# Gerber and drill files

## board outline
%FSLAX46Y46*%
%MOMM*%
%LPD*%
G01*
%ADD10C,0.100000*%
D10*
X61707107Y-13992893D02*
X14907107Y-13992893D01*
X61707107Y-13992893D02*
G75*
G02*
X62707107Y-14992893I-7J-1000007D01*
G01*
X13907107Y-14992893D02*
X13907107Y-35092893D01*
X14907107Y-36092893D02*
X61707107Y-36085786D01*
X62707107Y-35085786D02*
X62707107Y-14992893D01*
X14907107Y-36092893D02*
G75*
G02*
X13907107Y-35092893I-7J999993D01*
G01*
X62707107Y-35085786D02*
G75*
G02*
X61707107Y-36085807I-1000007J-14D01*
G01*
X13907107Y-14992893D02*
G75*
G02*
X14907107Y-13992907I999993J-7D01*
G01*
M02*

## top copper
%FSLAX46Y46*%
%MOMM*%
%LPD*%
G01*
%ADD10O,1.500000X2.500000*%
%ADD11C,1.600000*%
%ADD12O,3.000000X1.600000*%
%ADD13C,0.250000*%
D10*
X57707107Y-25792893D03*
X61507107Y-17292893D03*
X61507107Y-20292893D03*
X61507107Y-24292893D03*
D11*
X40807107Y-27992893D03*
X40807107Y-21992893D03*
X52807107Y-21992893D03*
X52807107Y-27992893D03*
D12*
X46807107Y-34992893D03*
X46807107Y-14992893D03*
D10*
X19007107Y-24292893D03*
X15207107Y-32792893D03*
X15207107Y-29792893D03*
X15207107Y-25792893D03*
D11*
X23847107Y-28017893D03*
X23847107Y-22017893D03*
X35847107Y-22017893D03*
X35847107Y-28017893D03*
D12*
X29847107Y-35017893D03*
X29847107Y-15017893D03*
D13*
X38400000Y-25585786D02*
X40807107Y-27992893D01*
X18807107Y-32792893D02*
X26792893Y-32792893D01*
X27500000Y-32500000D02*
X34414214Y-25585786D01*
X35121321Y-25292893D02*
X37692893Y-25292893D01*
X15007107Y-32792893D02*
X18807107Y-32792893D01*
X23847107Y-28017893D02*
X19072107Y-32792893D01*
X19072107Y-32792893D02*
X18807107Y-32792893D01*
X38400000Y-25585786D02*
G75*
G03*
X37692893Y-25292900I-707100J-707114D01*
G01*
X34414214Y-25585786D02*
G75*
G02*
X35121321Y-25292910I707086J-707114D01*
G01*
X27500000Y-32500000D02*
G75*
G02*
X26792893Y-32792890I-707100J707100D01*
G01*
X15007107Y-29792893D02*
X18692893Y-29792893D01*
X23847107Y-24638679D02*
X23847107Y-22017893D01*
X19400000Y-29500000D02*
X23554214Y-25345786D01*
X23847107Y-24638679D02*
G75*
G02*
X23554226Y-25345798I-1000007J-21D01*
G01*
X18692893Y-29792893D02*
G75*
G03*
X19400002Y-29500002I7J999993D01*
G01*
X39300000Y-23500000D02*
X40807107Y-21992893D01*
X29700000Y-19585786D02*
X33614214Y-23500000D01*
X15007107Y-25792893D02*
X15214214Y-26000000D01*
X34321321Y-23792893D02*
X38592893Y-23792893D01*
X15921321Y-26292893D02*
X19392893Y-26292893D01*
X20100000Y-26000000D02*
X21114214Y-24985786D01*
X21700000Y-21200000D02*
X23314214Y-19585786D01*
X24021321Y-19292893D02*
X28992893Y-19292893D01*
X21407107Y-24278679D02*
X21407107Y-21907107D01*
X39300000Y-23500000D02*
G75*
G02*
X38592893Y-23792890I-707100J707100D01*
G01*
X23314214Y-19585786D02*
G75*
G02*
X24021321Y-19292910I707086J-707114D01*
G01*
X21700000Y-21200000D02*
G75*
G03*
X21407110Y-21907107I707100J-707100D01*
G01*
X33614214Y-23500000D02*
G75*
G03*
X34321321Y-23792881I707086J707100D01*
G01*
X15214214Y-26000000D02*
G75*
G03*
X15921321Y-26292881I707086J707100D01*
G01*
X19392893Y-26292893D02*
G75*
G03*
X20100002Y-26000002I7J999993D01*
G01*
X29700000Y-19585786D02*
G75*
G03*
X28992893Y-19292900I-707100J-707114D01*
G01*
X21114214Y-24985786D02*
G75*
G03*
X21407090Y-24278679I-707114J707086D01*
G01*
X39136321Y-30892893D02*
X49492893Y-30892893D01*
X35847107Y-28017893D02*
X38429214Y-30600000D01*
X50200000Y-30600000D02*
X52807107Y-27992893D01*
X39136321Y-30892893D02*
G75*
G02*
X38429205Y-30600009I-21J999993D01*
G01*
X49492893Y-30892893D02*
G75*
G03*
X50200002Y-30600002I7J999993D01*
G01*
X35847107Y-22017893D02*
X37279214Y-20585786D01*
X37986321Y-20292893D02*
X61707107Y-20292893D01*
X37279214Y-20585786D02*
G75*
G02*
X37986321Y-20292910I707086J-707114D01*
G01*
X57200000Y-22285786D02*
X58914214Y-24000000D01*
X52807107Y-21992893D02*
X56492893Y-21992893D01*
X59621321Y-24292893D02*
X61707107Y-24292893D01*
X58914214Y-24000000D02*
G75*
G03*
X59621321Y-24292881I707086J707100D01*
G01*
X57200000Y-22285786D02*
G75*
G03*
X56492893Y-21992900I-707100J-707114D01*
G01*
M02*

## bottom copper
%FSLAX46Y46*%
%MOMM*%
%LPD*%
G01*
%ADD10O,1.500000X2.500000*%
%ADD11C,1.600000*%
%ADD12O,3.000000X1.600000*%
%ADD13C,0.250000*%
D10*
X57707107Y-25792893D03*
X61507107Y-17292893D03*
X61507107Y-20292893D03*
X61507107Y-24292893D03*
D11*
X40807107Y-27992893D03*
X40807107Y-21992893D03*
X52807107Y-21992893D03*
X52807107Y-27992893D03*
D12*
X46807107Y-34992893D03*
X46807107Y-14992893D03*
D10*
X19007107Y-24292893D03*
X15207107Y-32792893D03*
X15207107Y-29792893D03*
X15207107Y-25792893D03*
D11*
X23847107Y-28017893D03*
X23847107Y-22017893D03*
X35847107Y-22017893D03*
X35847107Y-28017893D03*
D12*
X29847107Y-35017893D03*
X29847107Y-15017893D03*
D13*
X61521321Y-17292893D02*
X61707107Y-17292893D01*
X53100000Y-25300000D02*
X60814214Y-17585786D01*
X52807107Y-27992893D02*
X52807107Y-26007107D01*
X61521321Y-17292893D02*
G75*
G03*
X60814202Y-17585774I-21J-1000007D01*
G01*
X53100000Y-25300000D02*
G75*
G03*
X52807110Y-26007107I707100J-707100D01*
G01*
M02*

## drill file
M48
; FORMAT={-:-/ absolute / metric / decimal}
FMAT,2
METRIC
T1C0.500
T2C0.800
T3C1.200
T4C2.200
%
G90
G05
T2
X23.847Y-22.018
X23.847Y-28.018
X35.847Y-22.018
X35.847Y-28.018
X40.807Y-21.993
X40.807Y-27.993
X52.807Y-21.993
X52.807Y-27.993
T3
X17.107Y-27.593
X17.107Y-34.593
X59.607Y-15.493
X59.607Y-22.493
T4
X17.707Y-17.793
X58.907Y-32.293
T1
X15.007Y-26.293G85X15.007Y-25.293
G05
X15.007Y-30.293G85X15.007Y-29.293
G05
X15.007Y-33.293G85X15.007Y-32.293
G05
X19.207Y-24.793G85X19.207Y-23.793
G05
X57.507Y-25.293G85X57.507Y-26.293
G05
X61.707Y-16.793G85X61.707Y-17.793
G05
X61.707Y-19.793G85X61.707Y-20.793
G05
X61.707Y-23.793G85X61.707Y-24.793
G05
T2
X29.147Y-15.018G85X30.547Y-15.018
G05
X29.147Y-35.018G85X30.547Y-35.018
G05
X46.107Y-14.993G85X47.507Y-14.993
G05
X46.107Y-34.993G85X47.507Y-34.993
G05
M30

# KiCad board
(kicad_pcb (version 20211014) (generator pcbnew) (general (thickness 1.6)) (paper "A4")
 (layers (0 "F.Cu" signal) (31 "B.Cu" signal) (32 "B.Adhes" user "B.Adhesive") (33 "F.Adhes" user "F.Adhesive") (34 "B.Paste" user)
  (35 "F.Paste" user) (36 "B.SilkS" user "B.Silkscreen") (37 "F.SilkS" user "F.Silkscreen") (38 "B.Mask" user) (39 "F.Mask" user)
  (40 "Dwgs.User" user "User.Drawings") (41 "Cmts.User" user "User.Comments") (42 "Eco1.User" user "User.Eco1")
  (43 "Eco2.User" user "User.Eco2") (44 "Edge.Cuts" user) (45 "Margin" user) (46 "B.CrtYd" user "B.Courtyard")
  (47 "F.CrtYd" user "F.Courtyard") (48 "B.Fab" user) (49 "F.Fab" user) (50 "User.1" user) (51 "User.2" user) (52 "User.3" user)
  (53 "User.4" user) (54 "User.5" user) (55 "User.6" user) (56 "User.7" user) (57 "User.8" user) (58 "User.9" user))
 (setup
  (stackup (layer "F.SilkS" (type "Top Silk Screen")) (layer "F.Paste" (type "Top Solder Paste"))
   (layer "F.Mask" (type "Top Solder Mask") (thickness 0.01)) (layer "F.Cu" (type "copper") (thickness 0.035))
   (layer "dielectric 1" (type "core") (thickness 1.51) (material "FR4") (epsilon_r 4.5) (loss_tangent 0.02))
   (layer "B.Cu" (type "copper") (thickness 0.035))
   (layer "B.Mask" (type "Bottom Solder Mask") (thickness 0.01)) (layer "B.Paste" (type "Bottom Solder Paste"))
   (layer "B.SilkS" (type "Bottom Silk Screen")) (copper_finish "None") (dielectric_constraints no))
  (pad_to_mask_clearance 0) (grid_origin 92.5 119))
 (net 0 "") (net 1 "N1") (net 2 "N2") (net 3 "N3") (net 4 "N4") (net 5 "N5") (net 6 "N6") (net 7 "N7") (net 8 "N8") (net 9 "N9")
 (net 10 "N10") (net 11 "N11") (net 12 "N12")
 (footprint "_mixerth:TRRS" (layer "F.Cu") (at 59.607107 13.992893)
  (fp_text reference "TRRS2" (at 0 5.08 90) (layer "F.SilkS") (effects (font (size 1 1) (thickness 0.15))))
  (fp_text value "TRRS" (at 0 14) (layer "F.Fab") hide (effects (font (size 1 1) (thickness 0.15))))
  (pad "" np_thru_hole circle (at 0 1.5) (size 1.2 1.2) (drill 1.2) (layers *.Cu *.Mask))
  (pad "" np_thru_hole circle (at 0 8.5) (size 1.2 1.2) (drill 1.2) (layers *.Cu *.Mask))
  (pad "A" thru_hole oval (at -2.1 11.8) (size 1.5 2.5) (drill oval 0.5 1.5 (offset 0.2 0)) (layers *.Cu "B.Mask") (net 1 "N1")
   (clearance 0.15))
  (pad "B" thru_hole oval (at 2.1 3.3) (size 1.5 2.5) (drill oval 0.5 1.5 (offset -0.2 0)) (layers *.Cu "B.Mask") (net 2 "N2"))
  (pad "C" thru_hole oval (at 2.1 6.3) (size 1.5 2.5) (drill oval 0.5 1.5 (offset -0.2 0)) (layers *.Cu "B.Mask") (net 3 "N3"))
  (pad "D" thru_hole oval (at 2.1 10.3) (size 1.5 2.5) (drill oval 0.5 1.5 (offset -0.2 0)) (layers *.Cu "B.Mask") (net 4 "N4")
   (clearance 0.15)))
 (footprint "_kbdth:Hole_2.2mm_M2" (layer "F.Cu") (at 58.907107 32.292893 90)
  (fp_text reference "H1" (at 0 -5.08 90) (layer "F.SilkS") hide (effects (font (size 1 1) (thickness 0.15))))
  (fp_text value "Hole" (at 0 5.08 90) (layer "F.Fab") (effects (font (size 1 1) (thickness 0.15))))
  (pad "" np_thru_hole circle locked (at 0 0 90) (size 2.2 2.2) (drill 2.2) (layers *.Cu *.Mask)))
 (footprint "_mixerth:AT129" (layer "F.Cu") (at 46.807107 24.992893 90)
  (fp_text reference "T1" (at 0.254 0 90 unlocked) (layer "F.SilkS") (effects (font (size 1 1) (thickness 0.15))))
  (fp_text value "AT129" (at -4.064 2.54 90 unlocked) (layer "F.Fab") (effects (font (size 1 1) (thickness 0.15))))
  (pad "1" thru_hole circle (at -3 -6 90) (size 1.6 1.6) (drill 0.8) (layers *.Cu "B.Mask") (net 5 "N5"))
  (pad "2" thru_hole circle (at 3 -6 90) (size 1.6 1.6) (drill 0.8) (layers *.Cu "B.Mask") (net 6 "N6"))
  (pad "3" thru_hole circle (at 3 6 90) (size 1.6 1.6) (drill 0.8) (layers *.Cu "B.Mask") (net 4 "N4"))
  (pad "4" thru_hole circle (at -3 6 90) (size 1.6 1.6) (drill 0.8) (layers *.Cu "B.Mask") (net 2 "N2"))
  (pad "5" thru_hole oval (at -10 0 90) (size 1.6 3) (drill oval 0.8 2.2) (layers *.Cu "B.Mask") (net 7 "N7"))
  (pad "6" thru_hole oval (at 10 0 90) (size 1.6 3) (drill oval 0.8 2.2) (layers *.Cu "B.Mask") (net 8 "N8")))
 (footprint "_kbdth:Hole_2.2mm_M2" (layer "F.Cu") (at 17.707107 17.792893 90)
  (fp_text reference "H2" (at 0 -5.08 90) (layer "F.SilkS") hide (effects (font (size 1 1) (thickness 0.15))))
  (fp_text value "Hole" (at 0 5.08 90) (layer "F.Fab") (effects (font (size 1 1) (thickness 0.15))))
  (pad "" np_thru_hole circle locked (at 0 0 90) (size 2.2 2.2) (drill 2.2) (layers *.Cu *.Mask)))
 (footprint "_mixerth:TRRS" (layer "F.Cu") (at 17.107107 36.092893 180)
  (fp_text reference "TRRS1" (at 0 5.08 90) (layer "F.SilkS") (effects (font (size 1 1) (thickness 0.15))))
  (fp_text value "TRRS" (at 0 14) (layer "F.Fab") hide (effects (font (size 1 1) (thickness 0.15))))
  (pad "" np_thru_hole circle (at 0 8.5 180) (size 1.2 1.2) (drill 1.2) (layers *.Cu *.Mask))
  (pad "" np_thru_hole circle (at 0 1.5 180) (size 1.2 1.2) (drill 1.2) (layers *.Cu *.Mask))
  (pad "A" thru_hole oval (at -2.1 11.8 180) (size 1.5 2.5) (drill oval 0.5 1.5 (offset 0.2 0)) (layers *.Cu "B.Mask") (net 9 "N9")
   (clearance 0.15))
  (pad "B" thru_hole oval (at 2.1 3.3 180) (size 1.5 2.5) (drill oval 0.5 1.5 (offset -0.2 0)) (layers *.Cu "B.Mask") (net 5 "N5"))
  (pad "C" thru_hole oval (at 2.1 6.3 180) (size 1.5 2.5) (drill oval 0.5 1.5 (offset -0.2 0)) (layers *.Cu "B.Mask") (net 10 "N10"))
  (pad "D" thru_hole oval (at 2.1 10.3 180) (size 1.5 2.5) (drill oval 0.5 1.5 (offset -0.2 0)) (layers *.Cu "B.Mask") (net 6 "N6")
   (clearance 0.15)))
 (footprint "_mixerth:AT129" (layer "F.Cu") (at 29.847107 25.017893 90)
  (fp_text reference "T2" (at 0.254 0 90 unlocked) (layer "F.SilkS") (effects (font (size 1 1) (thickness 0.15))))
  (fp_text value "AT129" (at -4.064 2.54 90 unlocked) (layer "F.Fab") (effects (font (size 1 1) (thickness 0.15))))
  (pad "1" thru_hole circle (at -3 -6 90) (size 1.6 1.6) (drill 0.8) (layers *.Cu "B.Mask") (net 5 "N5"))
  (pad "2" thru_hole circle (at 3 -6 90) (size 1.6 1.6) (drill 0.8) (layers *.Cu "B.Mask") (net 10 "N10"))
  (pad "3" thru_hole circle (at 3 6 90) (size 1.6 1.6) (drill 0.8) (layers *.Cu "B.Mask") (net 3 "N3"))
  (pad "4" thru_hole circle (at -3 6 90) (size 1.6 1.6) (drill 0.8) (layers *.Cu "B.Mask") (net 2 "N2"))
  (pad "5" thru_hole oval (at -10 0 90) (size 1.6 3) (drill oval 0.8 2.2) (layers *.Cu "B.Mask") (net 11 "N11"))
  (pad "6" thru_hole oval (at 10 0 90) (size 1.6 3) (drill oval 0.8 2.2) (layers *.Cu "B.Mask") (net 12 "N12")))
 (gr_line (start 61.707107 13.992893) (end 14.907107 13.992893) (layer "Edge.Cuts") (width 0.1))
 (gr_arc (start 61.707107 13.992893) (mid 62.414214 14.285786) (end 62.707107 14.992893) (layer "Edge.Cuts") (width 0.1))
 (gr_line (start 13.907107 14.992893) (end 13.907107 35.092893) (layer "Edge.Cuts") (width 0.1))
 (gr_line (start 14.907107 36.092893) (end 61.707107 36.085786) (layer "Edge.Cuts") (width 0.1))
 (gr_line (start 62.707107 35.085786) (end 62.707107 14.992893) (layer "Edge.Cuts") (width 0.1))
 (gr_arc (start 14.907107 36.092893) (mid 14.2 35.8) (end 13.907107 35.092893) (layer "Edge.Cuts") (width 0.1))
 (gr_arc (start 62.707107 35.085786) (mid 62.414216 35.792897) (end 61.707107 36.085786) (layer "Edge.Cuts") (width 0.1))
 (gr_arc (start 13.907107 14.992893) (mid 14.2 14.285786) (end 14.907107 13.992893) (layer "Edge.Cuts") (width 0.1))
 (segment (start 38.4 25.585786) (end 40.807107 27.992893) (width 0.25) (layer "F.Cu") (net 5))
 (segment (start 18.807107 32.792893) (end 26.792893 32.792893) (width 0.25) (layer "F.Cu") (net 5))
 (segment (start 27.5 32.5) (end 34.414214 25.585786) (width 0.25) (layer "F.Cu") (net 5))
 (segment (start 35.121321 25.292893) (end 37.692893 25.292893) (width 0.25) (layer "F.Cu") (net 5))
 (segment (start 15.007107 32.792893) (end 18.807107 32.792893) (width 0.25) (layer "F.Cu") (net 5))
 (segment (start 23.847107 28.017893) (end 19.072107 32.792893) (width 0.25) (layer "F.Cu") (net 5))
 (segment (start 19.072107 32.792893) (end 18.807107 32.792893) (width 0.25) (layer "F.Cu") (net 5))
 (arc (start 38.4 25.585786) (mid 38.075577 25.369013) (end 37.692893 25.292893) (width 0.25) (layer "F.Cu") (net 5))
 (arc (start 34.414214 25.585786) (mid 34.738637 25.369013) (end 35.121321 25.292893) (width 0.25) (layer "F.Cu") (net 5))
 (arc (start 27.5 32.5) (mid 27.175577 32.716773) (end 26.792893 32.792893) (width 0.25) (layer "F.Cu") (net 5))
 (segment (start 15.007107 29.792893) (end 18.692893 29.792893) (width 0.25) (layer "F.Cu") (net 10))
 (segment (start 23.847107 24.638679) (end 23.847107 22.017893) (width 0.25) (layer "F.Cu") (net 10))
 (segment (start 19.4 29.5) (end 23.554214 25.345786) (width 0.25) (layer "F.Cu") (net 10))
 (arc (start 23.847107 24.638679) (mid 23.770987 25.021362) (end 23.554214 25.345786) (width 0.25) (layer "F.Cu") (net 10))
 (arc (start 18.692893 29.792893) (mid 19.075576 29.716773) (end 19.4 29.5) (width 0.25) (layer "F.Cu") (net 10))
 (segment (start 39.3 23.5) (end 40.807107 21.992893) (width 0.25) (layer "F.Cu") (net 6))
 (segment (start 29.7 19.585786) (end 33.614214 23.5) (width 0.25) (layer "F.Cu") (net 6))
 (segment (start 15.007107 25.792893) (end 15.214214 26) (width 0.25) (layer "F.Cu") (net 6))
 (segment (start 34.321321 23.792893) (end 38.592893 23.792893) (width 0.25) (layer "F.Cu") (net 6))
 (segment (start 15.921321 26.292893) (end 19.392893 26.292893) (width 0.25) (layer "F.Cu") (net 6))
 (segment (start 20.1 26) (end 21.114214 24.985786) (width 0.25) (layer "F.Cu") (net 6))
 (segment (start 21.7 21.2) (end 23.314214 19.585786) (width 0.25) (layer "F.Cu") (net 6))
 (segment (start 24.021321 19.292893) (end 28.992893 19.292893) (width 0.25) (layer "F.Cu") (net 6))
 (segment (start 21.407107 24.278679) (end 21.407107 21.907107) (width 0.25) (layer "F.Cu") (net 6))
 (arc (start 39.3 23.5) (mid 38.975577 23.716773) (end 38.592893 23.792893) (width 0.25) (layer "F.Cu") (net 6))
 (arc (start 23.314214 19.585786) (mid 23.638637 19.369013) (end 24.021321 19.292893) (width 0.25) (layer "F.Cu") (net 6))
 (arc (start 21.7 21.2) (mid 21.483227 21.524423) (end 21.407107 21.907107) (width 0.25) (layer "F.Cu") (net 6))
 (arc (start 33.614214 23.5) (mid 33.938637 23.716773) (end 34.321321 23.792893) (width 0.25) (layer "F.Cu") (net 6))
 (arc (start 15.214214 26) (mid 15.538637 26.216773) (end 15.921321 26.292893) (width 0.25) (layer "F.Cu") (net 6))
 (arc (start 19.392893 26.292893) (mid 19.775576 26.216773) (end 20.1 26) (width 0.25) (layer "F.Cu") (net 6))
 (arc (start 29.7 19.585786) (mid 29.375577 19.369013) (end 28.992893 19.292893) (width 0.25) (layer "F.Cu") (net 6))
 (arc (start 21.114214 24.985786) (mid 21.330987 24.661363) (end 21.407107 24.278679) (width 0.25) (layer "F.Cu") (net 6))
 (segment (start 39.136321 30.892893) (end 49.492893 30.892893) (width 0.25) (layer "F.Cu") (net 2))
 (segment (start 35.847107 28.017893) (end 38.429214 30.6) (width 0.25) (layer "F.Cu") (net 2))
 (segment (start 50.2 30.6) (end 52.807107 27.992893) (width 0.25) (layer "F.Cu") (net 2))
 (arc (start 39.136321 30.892893) (mid 38.753638 30.816773) (end 38.429214 30.6) (width 0.25) (layer "F.Cu") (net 2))
 (arc (start 49.492893 30.892893) (mid 49.875576 30.816773) (end 50.2 30.6) (width 0.25) (layer "F.Cu") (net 2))
 (segment (start 61.521321 17.292893) (end 61.707107 17.292893) (width 0.25) (layer "B.Cu") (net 2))
 (segment (start 53.1 25.3) (end 60.814214 17.585786) (width 0.25) (layer "B.Cu") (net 2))
 (segment (start 52.807107 27.992893) (end 52.807107 26.007107) (width 0.25) (layer "B.Cu") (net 2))
 (arc (start 61.521321 17.292893) (mid 61.138638 17.369013) (end 60.814214 17.585786) (width 0.25) (layer "B.Cu") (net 2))
 (arc (start 53.1 25.3) (mid 52.883227 25.624423) (end 52.807107 26.007107) (width 0.25) (layer "B.Cu") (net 2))
 (segment (start 35.847107 22.017893) (end 37.279214 20.585786) (width 0.25) (layer "F.Cu") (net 3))
 (segment (start 37.986321 20.292893) (end 61.707107 20.292893) (width 0.25) (layer "F.Cu") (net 3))
 (arc (start 37.279214 20.585786) (mid 37.603637 20.369013) (end 37.986321 20.292893) (width 0.25) (layer "F.Cu") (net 3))
 (segment (start 57.2 22.285786) (end 58.914214 24) (width 0.25) (layer "F.Cu") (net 4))
 (segment (start 52.807107 21.992893) (end 56.492893 21.992893) (width 0.25) (layer "F.Cu") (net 4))
 (segment (start 59.621321 24.292893) (end 61.707107 24.292893) (width 0.25) (layer "F.Cu") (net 4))
 (arc (start 58.914214 24) (mid 59.238637 24.216773) (end 59.621321 24.292893) (width 0.25) (layer "F.Cu") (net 4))
 (arc (start 57.2 22.285786) (mid 56.875577 22.069013) (end 56.492893 21.992893) (width 0.25) (layer "F.Cu") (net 4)))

